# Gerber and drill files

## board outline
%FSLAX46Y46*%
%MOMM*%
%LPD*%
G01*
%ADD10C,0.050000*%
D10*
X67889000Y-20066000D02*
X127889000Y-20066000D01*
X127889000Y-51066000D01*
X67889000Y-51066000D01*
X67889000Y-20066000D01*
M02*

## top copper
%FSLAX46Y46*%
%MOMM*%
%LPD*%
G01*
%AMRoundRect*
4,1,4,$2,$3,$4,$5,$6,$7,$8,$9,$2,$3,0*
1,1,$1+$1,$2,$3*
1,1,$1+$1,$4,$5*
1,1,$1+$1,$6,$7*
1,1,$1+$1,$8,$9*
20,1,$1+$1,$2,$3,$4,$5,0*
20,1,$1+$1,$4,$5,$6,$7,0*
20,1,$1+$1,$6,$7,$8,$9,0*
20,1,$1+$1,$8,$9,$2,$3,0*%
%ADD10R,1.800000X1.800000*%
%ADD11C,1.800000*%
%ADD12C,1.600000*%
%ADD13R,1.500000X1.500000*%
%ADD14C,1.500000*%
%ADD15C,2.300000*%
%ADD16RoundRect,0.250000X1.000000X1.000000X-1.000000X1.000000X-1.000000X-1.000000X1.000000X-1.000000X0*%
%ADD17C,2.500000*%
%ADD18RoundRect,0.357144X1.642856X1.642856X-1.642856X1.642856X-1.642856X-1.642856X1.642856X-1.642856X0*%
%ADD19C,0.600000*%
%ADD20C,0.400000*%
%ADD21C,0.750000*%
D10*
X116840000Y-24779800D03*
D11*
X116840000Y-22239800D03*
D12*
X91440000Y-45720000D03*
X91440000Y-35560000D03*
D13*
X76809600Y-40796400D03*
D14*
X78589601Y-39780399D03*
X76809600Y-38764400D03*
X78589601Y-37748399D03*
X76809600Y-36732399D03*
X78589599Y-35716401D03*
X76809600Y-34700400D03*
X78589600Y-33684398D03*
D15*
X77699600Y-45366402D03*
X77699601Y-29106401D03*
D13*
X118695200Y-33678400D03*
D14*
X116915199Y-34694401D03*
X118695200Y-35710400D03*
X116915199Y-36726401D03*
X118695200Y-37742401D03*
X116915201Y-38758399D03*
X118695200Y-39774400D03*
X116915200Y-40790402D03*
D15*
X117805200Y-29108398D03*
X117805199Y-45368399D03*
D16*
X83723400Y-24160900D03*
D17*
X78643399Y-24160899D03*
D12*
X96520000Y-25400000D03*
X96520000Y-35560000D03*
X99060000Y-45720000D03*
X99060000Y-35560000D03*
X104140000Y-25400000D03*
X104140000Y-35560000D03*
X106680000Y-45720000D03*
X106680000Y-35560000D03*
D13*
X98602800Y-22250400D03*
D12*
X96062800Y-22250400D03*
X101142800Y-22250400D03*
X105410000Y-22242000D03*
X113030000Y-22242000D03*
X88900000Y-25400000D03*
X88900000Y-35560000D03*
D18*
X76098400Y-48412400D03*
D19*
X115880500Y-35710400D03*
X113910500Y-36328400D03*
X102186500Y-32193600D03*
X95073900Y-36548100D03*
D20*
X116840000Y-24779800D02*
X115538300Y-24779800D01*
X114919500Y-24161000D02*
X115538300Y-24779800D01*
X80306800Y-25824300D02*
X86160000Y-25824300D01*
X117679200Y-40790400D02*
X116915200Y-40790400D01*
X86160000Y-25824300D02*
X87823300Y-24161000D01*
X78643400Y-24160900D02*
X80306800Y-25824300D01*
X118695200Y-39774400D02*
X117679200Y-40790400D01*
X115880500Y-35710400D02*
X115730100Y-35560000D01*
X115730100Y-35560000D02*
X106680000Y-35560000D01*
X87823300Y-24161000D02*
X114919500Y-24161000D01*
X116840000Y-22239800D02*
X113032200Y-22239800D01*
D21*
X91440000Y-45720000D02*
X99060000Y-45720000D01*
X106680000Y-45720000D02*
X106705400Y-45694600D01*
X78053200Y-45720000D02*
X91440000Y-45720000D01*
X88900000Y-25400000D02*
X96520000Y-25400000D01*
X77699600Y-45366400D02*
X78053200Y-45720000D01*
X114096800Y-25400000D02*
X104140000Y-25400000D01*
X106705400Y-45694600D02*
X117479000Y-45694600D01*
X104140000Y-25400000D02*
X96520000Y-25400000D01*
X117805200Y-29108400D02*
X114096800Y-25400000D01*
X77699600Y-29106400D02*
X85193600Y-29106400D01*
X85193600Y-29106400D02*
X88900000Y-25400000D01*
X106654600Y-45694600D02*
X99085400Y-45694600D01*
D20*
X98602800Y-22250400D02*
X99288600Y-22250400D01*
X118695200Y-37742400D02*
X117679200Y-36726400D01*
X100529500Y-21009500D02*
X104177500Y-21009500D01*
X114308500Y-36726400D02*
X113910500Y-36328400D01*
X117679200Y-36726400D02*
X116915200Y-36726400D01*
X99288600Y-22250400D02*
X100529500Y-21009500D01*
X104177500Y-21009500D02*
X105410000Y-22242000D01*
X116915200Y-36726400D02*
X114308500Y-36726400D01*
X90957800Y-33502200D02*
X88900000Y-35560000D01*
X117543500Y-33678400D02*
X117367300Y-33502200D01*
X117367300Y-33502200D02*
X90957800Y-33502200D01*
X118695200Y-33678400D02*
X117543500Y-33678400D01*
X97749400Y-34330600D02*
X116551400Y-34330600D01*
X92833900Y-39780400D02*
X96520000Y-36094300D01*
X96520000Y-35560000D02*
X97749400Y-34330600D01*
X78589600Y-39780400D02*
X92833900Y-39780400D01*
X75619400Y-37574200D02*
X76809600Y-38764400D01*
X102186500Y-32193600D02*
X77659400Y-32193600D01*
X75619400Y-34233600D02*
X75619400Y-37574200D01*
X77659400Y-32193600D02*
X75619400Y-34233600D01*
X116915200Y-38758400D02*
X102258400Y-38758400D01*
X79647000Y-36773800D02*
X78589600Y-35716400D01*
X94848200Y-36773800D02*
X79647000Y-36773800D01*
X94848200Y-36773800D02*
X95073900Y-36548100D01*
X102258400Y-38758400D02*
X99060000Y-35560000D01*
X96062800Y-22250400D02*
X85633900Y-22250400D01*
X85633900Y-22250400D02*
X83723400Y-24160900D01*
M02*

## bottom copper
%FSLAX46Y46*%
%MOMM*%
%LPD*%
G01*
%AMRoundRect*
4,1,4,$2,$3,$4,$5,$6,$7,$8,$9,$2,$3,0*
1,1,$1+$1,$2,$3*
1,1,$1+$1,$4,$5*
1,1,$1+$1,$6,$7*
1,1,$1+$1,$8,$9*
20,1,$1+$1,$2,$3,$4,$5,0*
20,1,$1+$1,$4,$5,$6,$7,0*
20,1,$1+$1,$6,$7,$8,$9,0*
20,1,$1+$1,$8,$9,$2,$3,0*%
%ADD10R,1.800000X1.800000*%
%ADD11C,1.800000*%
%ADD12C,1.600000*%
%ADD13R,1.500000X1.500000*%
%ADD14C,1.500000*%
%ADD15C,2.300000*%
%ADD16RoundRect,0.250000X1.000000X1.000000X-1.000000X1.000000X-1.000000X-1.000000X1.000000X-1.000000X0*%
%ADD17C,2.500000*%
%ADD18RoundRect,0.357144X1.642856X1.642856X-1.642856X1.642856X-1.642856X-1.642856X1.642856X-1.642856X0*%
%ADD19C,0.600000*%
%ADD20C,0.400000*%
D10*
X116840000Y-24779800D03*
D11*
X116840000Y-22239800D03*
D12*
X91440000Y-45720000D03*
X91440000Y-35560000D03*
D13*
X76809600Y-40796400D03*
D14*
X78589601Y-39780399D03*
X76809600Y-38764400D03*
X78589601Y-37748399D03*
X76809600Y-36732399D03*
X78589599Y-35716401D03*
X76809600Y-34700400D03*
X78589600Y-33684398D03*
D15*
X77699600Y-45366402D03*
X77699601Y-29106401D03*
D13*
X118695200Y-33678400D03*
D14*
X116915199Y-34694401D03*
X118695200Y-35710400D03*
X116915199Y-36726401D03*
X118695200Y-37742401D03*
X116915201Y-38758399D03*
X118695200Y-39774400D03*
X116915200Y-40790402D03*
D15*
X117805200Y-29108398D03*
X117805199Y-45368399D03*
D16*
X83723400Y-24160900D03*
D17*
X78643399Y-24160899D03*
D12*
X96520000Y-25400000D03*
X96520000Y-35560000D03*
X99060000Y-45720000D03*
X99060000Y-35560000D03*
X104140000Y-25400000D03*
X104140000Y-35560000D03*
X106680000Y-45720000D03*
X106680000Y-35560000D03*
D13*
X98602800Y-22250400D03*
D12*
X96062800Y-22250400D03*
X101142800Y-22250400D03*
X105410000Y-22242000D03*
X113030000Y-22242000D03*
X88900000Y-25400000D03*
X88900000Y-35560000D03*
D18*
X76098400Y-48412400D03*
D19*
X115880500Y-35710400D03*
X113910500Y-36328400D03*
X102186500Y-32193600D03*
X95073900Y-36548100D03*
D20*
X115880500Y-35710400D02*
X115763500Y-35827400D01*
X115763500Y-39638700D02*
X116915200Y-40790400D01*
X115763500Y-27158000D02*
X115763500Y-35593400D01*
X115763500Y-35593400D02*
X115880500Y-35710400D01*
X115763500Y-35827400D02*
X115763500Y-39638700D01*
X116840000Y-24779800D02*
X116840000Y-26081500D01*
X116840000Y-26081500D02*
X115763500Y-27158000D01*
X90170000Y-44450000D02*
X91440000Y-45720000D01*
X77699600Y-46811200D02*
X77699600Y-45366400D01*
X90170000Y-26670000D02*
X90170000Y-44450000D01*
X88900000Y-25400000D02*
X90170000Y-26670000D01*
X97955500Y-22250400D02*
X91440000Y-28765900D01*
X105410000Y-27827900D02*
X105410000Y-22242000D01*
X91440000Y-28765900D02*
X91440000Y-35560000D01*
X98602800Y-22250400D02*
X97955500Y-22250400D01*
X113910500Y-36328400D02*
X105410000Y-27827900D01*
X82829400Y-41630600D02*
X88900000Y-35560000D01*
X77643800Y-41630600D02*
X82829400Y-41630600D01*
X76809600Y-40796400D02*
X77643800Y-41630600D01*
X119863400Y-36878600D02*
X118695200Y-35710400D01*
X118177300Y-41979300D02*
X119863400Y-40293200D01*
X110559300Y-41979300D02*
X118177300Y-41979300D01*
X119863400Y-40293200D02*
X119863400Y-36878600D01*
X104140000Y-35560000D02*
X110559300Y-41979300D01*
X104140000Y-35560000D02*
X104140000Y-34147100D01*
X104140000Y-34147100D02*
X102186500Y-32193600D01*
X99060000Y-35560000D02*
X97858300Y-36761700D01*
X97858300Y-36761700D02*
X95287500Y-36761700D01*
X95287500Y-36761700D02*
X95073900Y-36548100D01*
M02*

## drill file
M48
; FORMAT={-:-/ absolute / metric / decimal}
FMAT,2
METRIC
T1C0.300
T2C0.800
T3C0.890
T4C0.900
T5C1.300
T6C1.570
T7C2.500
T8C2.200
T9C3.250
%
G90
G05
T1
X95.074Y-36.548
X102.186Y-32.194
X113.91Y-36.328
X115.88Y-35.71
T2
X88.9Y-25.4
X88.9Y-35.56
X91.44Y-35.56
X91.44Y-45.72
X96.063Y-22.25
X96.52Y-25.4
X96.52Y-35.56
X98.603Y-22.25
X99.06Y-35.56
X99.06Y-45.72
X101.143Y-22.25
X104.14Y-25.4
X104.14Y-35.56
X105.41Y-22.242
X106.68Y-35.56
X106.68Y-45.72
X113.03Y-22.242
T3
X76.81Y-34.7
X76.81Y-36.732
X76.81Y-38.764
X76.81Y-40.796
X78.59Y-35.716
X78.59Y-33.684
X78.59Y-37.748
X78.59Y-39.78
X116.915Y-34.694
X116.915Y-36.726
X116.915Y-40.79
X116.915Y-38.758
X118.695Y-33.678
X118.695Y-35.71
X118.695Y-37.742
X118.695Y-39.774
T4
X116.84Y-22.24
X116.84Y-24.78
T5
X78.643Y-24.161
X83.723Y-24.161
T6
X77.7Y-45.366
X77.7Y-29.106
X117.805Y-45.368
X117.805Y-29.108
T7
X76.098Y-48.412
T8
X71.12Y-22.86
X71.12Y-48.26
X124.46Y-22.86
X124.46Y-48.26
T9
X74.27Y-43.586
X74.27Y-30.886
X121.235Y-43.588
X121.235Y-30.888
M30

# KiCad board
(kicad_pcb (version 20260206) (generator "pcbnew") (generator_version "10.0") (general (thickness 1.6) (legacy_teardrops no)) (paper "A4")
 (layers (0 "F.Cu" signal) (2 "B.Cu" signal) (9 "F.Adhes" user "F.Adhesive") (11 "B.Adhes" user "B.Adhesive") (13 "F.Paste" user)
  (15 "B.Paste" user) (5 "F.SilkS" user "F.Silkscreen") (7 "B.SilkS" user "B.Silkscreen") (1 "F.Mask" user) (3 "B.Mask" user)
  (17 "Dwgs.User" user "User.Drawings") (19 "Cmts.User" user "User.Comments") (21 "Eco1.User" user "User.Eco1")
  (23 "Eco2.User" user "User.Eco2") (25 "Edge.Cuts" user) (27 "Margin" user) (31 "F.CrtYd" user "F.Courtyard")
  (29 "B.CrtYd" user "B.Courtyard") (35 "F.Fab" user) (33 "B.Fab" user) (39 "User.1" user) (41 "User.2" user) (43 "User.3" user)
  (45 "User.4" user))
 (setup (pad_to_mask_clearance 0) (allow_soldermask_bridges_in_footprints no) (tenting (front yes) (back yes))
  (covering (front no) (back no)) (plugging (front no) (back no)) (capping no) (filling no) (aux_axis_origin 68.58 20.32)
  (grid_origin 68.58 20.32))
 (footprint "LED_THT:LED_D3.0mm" (layer "F.Cu") (at 116.84 24.7798 90)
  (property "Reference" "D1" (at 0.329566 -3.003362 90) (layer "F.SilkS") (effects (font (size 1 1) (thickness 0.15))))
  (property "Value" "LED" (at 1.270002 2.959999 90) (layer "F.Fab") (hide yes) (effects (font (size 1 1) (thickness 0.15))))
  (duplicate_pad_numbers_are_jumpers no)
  (pad "1" thru_hole rect (at 0 0 90) (size 1.8 1.8) (drill 0.9) (layers "*.Cu" "*.Mask") (remove_unused_layers no) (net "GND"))
  (pad "2" thru_hole circle (at 2.54 0 90) (size 1.8 1.8) (drill 0.9) (layers "*.Cu" "*.Mask") (remove_unused_layers no) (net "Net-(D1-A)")))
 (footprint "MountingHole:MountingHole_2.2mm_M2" (layer "F.Cu") (at 124.46 22.86)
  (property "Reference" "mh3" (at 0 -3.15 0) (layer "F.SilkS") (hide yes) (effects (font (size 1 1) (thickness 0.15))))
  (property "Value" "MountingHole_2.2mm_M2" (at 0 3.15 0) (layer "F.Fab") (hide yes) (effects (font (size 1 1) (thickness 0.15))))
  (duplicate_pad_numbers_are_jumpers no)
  (pad "" np_thru_hole circle (at 0 0) (size 2.2 2.2) (drill 2.2) (layers "*.Cu" "*.Mask")))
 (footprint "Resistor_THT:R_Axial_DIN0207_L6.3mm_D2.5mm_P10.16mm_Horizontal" (layer "F.Cu") (at 91.44 45.72 90)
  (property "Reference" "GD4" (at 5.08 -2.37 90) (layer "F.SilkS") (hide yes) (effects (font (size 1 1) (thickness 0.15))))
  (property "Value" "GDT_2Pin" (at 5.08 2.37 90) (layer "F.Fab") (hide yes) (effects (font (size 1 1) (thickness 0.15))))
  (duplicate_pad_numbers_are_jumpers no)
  (pad "1" thru_hole circle (at 0 0 90) (size 1.6 1.6) (drill 0.8) (layers "*.Cu" "*.Mask") (remove_unused_layers no) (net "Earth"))
  (pad "2" thru_hole circle (at 10.16 0 90) (size 1.6 1.6) (drill 0.8) (layers "*.Cu" "*.Mask") (remove_unused_layers no)
   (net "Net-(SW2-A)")))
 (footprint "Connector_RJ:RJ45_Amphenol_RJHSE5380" (layer "F.Cu") (at 76.8096 40.7964 90)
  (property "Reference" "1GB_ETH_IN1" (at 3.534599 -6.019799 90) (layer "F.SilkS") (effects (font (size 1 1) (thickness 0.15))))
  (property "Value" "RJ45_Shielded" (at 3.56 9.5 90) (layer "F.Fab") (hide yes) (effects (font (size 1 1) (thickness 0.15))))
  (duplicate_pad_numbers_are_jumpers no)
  (pad "" np_thru_hole circle (at -2.79 -2.54 90) (size 3.25 3.25) (drill 3.25) (layers "*.Cu" "*.Mask"))
  (pad "" np_thru_hole circle (at 9.909999 -2.539999 90) (size 3.25 3.25) (drill 3.25) (layers "*.Cu" "*.Mask"))
  (pad "1" thru_hole rect (at 0 0 90) (size 1.5 1.5) (drill 0.89) (layers "*.Cu" "*.Mask") (remove_unused_layers no)
   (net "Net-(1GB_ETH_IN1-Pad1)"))
  (pad "2" thru_hole circle (at 1.016001 1.780001 90) (size 1.5 1.5) (drill 0.89) (layers "*.Cu" "*.Mask") (remove_unused_layers no)
   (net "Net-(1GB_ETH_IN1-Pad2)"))
  (pad "3" thru_hole circle (at 2.032 0 90) (size 1.5 1.5) (drill 0.89) (layers "*.Cu" "*.Mask") (remove_unused_layers no)
   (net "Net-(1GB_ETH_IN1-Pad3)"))
  (pad "4" thru_hole circle (at 3.048001 1.780001 90) (size 1.5 1.5) (drill 0.89) (layers "*.Cu" "*.Mask") (remove_unused_layers no)
   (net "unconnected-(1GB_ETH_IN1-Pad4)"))
  (pad "5" thru_hole circle (at 4.064001 0 90) (size 1.5 1.5) (drill 0.89) (layers "*.Cu" "*.Mask") (remove_unused_layers no)
   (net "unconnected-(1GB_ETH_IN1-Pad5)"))
  (pad "6" thru_hole circle (at 5.079999 1.779999 90) (size 1.5 1.5) (drill 0.89) (layers "*.Cu" "*.Mask") (remove_unused_layers no)
   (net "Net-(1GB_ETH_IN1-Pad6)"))
  (pad "7" thru_hole circle (at 6.096 0 90) (size 1.5 1.5) (drill 0.89) (layers "*.Cu" "*.Mask") (remove_unused_layers no)
   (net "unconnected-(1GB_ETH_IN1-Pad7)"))
  (pad "8" thru_hole circle (at 7.112002 1.78 90) (size 1.5 1.5) (drill 0.89) (layers "*.Cu" "*.Mask") (remove_unused_layers no)
   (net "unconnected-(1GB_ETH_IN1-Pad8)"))
  (pad "SH" thru_hole circle (at -4.570002 0.89 90) (size 2.3 2.3) (drill 1.57) (layers "*.Cu" "*.Mask") (remove_unused_layers no)
   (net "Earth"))
  (pad "SH" thru_hole circle (at 11.689999 0.890001 90) (size 2.3 2.3) (drill 1.57) (layers "*.Cu" "*.Mask") (remove_unused_layers no)
   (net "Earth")))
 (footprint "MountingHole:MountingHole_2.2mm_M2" (layer "F.Cu") (at 124.46 48.26)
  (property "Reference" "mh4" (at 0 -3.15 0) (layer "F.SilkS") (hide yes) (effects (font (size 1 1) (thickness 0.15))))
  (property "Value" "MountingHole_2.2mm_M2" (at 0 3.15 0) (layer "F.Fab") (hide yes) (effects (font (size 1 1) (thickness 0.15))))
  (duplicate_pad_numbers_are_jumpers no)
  (pad "" np_thru_hole circle (at 0 0) (size 2.2 2.2) (drill 2.2) (layers "*.Cu" "*.Mask")))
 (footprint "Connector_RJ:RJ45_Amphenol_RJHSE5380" (layer "F.Cu") (at 118.6952 33.6784 -90)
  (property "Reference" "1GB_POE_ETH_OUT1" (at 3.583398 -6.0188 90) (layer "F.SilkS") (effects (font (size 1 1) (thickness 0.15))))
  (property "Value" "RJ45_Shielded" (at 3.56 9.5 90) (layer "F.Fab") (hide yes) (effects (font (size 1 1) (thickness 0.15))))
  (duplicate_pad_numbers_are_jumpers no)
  (pad "" np_thru_hole circle (at -2.79 -2.54 270) (size 3.25 3.25) (drill 3.25) (layers "*.Cu" "*.Mask"))
  (pad "" np_thru_hole circle (at 9.909999 -2.539999 270) (size 3.25 3.25) (drill 3.25) (layers "*.Cu" "*.Mask"))
  (pad "1" thru_hole rect (at 0 0 270) (size 1.5 1.5) (drill 0.89) (layers "*.Cu" "*.Mask") (remove_unused_layers no)
   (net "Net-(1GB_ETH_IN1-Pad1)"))
  (pad "2" thru_hole circle (at 1.016001 1.780001 270) (size 1.5 1.5) (drill 0.89) (layers "*.Cu" "*.Mask") (remove_unused_layers no)
   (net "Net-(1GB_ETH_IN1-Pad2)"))
  (pad "3" thru_hole circle (at 2.032 0 270) (size 1.5 1.5) (drill 0.89) (layers "*.Cu" "*.Mask") (remove_unused_layers no)
   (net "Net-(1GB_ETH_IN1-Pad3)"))
  (pad "4" thru_hole circle (at 3.048001 1.780001 270) (size 1.5 1.5) (drill 0.89) (layers "*.Cu" "*.Mask") (remove_unused_layers no)
   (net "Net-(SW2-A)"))
  (pad "5" thru_hole circle (at 4.064001 0 270) (size 1.5 1.5) (drill 0.89) (layers "*.Cu" "*.Mask") (remove_unused_layers no)
   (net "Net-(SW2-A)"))
  (pad "6" thru_hole circle (at 5.079999 1.779999 270) (size 1.5 1.5) (drill 0.89) (layers "*.Cu" "*.Mask") (remove_unused_layers no)
   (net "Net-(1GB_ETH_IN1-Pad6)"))
  (pad "7" thru_hole circle (at 6.096 0 270) (size 1.5 1.5) (drill 0.89) (layers "*.Cu" "*.Mask") (remove_unused_layers no) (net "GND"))
  (pad "8" thru_hole circle (at 7.112002 1.78 270) (size 1.5 1.5) (drill 0.89) (layers "*.Cu" "*.Mask") (remove_unused_layers no)
   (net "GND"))
  (pad "SH" thru_hole circle (at -4.570002 0.89 270) (size 2.3 2.3) (drill 1.57) (layers "*.Cu" "*.Mask") (remove_unused_layers no)
   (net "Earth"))
  (pad "SH" thru_hole circle (at 11.689999 0.890001 270) (size 2.3 2.3) (drill 1.57) (layers "*.Cu" "*.Mask") (remove_unused_layers no)
   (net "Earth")))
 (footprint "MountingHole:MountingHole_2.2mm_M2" (layer "F.Cu") (at 71.12 22.86)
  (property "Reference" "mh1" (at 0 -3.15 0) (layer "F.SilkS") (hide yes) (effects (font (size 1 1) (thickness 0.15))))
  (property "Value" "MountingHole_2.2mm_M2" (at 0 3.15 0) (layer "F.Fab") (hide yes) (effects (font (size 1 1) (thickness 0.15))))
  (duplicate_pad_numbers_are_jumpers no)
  (pad "" np_thru_hole circle (at 0 0) (size 2.2 2.2) (drill 2.2) (layers "*.Cu" "*.Mask")))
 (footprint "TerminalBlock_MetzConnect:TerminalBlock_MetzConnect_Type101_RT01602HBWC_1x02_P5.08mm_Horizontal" (layer "F.Cu")
  (at 83.7234 24.1609 180)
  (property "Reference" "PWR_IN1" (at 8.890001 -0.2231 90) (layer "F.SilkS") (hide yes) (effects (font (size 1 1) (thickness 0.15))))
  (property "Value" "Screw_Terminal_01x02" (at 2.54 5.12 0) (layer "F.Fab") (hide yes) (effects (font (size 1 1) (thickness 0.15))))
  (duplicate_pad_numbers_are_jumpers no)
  (pad "1" thru_hole roundrect (at 0 0 180) (size 2.5 2.5) (drill 1.3) (layers "*.Cu" "*.Mask") (remove_unused_layers no)
   (roundrect_rratio 0.1) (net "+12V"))
  (pad "2" thru_hole circle (at 5.080001 0.000001 180) (size 2.5 2.5) (drill 1.3) (layers "*.Cu" "*.Mask") (remove_unused_layers no)
   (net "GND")))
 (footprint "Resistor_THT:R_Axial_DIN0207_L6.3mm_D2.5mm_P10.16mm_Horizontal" (layer "F.Cu") (at 96.52 25.4 -90)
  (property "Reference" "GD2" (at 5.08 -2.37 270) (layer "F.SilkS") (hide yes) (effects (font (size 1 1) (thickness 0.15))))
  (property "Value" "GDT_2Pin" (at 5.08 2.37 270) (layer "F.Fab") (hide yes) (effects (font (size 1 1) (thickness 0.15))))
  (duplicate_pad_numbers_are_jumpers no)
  (pad "1" thru_hole circle (at 0 0 270) (size 1.6 1.6) (drill 0.8) (layers "*.Cu" "*.Mask") (remove_unused_layers no) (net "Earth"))
  (pad "2" thru_hole circle (at 10.16 0 270) (size 1.6 1.6) (drill 0.8) (layers "*.Cu" "*.Mask") (remove_unused_layers no)
   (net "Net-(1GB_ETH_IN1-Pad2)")))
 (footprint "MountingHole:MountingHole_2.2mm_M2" (layer "F.Cu") (at 71.12 48.26)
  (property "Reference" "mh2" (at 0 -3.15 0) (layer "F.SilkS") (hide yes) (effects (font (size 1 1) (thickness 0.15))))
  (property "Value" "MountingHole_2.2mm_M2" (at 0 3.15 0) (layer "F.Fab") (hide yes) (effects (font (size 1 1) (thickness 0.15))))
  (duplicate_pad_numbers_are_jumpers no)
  (pad "" np_thru_hole circle (at 0 0) (size 2.2 2.2) (drill 2.2) (layers "*.Cu" "*.Mask")))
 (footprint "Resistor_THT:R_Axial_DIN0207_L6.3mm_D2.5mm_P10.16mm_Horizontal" (layer "F.Cu") (at 99.06 45.72 90)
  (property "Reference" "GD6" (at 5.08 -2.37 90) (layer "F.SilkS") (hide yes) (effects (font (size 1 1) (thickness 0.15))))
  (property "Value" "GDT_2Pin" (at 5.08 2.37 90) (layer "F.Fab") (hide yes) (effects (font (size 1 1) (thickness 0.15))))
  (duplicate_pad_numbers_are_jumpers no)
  (pad "1" thru_hole circle (at 0 0 90) (size 1.6 1.6) (drill 0.8) (layers "*.Cu" "*.Mask") (remove_unused_layers no) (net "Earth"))
  (pad "2" thru_hole circle (at 10.16 0 90) (size 1.6 1.6) (drill 0.8) (layers "*.Cu" "*.Mask") (remove_unused_layers no)
   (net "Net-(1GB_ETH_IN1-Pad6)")))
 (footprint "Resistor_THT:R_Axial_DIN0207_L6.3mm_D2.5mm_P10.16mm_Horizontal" (layer "F.Cu") (at 104.14 25.4 -90)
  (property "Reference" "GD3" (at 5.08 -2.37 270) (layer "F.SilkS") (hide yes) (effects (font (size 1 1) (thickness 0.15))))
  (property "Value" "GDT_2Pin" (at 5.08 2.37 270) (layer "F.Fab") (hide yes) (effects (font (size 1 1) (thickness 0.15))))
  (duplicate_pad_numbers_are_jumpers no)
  (pad "1" thru_hole circle (at 0 0 270) (size 1.6 1.6) (drill 0.8) (layers "*.Cu" "*.Mask") (remove_unused_layers no) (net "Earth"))
  (pad "2" thru_hole circle (at 10.16 0 270) (size 1.6 1.6) (drill 0.8) (layers "*.Cu" "*.Mask") (remove_unused_layers no)
   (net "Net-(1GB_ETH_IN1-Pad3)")))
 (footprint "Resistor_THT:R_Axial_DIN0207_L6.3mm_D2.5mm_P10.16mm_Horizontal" (layer "F.Cu") (at 106.68 45.72 90)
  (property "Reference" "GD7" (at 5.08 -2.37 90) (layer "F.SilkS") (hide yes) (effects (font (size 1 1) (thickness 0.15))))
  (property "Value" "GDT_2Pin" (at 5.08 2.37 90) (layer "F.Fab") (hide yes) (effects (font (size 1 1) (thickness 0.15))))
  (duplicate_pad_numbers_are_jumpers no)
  (pad "1" thru_hole circle (at 0 0 90) (size 1.6 1.6) (drill 0.8) (layers "*.Cu" "*.Mask") (remove_unused_layers no) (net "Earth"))
  (pad "2" thru_hole circle (at 10.16 0 90) (size 1.6 1.6) (drill 0.8) (layers "*.Cu" "*.Mask") (remove_unused_layers no) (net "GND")))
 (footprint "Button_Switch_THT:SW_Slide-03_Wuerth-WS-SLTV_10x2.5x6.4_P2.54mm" (layer "F.Cu") (at 98.6028 22.2504)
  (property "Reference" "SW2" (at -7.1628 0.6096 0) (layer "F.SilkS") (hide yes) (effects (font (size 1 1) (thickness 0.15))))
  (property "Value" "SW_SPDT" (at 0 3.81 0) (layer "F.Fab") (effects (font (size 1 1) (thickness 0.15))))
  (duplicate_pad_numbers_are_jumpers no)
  (pad "1" thru_hole rect (at 0 0) (size 1.5 1.5) (drill 0.8) (layers "*.Cu" "*.Mask") (remove_unused_layers no) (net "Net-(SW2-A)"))
  (pad "2" thru_hole circle (at -2.54 0) (size 1.6 1.6) (drill 0.8) (layers "*.Cu" "*.Mask") (remove_unused_layers no) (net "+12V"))
  (pad "3" thru_hole circle (at 2.54 0) (size 1.6 1.6) (drill 0.8) (layers "*.Cu" "*.Mask") (remove_unused_layers no)
   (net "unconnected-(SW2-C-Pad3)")))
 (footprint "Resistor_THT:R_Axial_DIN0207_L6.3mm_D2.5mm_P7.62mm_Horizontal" (layer "F.Cu") (at 105.41 22.242)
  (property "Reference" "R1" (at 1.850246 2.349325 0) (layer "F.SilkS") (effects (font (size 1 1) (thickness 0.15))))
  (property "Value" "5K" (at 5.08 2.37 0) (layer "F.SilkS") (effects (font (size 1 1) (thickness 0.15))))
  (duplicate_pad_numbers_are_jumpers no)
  (pad "1" thru_hole circle (at 0 0) (size 1.6 1.6) (drill 0.8) (layers "*.Cu" "*.Mask") (remove_unused_layers no) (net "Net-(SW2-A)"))
  (pad "2" thru_hole circle (at 7.62 0) (size 1.6 1.6) (drill 0.8) (layers "*.Cu" "*.Mask") (remove_unused_layers no) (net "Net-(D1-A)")))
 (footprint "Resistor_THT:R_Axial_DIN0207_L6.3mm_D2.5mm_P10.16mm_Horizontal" (layer "F.Cu") (at 88.9 25.4 -90)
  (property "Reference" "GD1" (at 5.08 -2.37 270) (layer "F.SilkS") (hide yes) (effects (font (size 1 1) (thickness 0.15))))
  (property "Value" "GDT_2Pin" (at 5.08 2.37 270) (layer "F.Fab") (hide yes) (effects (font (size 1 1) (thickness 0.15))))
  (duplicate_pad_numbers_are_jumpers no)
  (pad "1" thru_hole circle (at 0 0 270) (size 1.6 1.6) (drill 0.8) (layers "*.Cu" "*.Mask") (remove_unused_layers no) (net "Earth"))
  (pad "2" thru_hole circle (at 10.16 0 270) (size 1.6 1.6) (drill 0.8) (layers "*.Cu" "*.Mask") (remove_unused_layers no)
   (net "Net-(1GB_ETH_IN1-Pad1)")))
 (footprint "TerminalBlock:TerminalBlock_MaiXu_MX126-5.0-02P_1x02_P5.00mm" (layer "B.Cu") (at 76.0984 48.4124 180)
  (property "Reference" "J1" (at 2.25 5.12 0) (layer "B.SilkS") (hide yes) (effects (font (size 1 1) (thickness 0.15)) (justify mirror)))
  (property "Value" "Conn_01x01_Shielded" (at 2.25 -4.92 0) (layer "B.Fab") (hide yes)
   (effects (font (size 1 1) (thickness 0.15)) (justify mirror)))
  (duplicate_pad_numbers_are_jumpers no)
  (pad "1" thru_hole roundrect (at 0 0 180) (size 4 4) (drill 2.5) (layers "*.Cu" "*.Mask") (remove_unused_layers yes) (keep_end_layers yes)
   (zone_layer_connections) (roundrect_rratio 0.089286) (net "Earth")))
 (gr_rect (start 67.889 20.066) (end 127.889 51.066) (stroke (width 0.05) (type solid)) (fill no) (layer "Edge.Cuts"))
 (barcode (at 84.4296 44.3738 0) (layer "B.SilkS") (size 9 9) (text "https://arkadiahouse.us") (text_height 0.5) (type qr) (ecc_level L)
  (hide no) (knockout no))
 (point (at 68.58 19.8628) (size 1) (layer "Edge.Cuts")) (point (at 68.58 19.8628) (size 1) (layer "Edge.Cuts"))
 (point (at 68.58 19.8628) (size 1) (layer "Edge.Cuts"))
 (segment (start 116.84 24.7798) (end 115.5383 24.7798) (width 0.4) (layer "F.Cu") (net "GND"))
 (segment (start 114.9195 24.161) (end 115.5383 24.7798) (width 0.4) (layer "F.Cu") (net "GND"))
 (segment (start 80.3068 25.8243) (end 86.16 25.8243) (width 0.4) (layer "F.Cu") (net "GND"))
 (segment (start 117.6792 40.7904) (end 116.9152 40.7904) (width 0.4) (layer "F.Cu") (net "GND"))
 (segment (start 86.16 25.8243) (end 87.8233 24.161) (width 0.4) (layer "F.Cu") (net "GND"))
 (segment (start 78.6434 24.1609) (end 80.3068 25.8243) (width 0.4) (layer "F.Cu") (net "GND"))
 (segment (start 118.6952 39.7744) (end 117.6792 40.7904) (width 0.4) (layer "F.Cu") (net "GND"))
 (segment (start 115.8805 35.7104) (end 115.7301 35.56) (width 0.4) (layer "F.Cu") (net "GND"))
 (segment (start 115.7301 35.56) (end 106.68 35.56) (width 0.4) (layer "F.Cu") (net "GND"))
 (segment (start 87.8233 24.161) (end 114.9195 24.161) (width 0.4) (layer "F.Cu") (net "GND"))
 (via (at 115.8805 35.7104) (size 0.6) (drill 0.3) (layers "F.Cu" "B.Cu") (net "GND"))
 (segment (start 115.8805 35.7104) (end 115.7635 35.8274) (width 0.4) (layer "B.Cu") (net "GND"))
 (segment (start 115.7635 39.6387) (end 116.9152 40.7904) (width 0.4) (layer "B.Cu") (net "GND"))
 (segment (start 115.7635 27.158) (end 115.7635 35.5934) (width 0.4) (layer "B.Cu") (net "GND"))
 (segment (start 115.7635 35.5934) (end 115.8805 35.7104) (width 0.4) (layer "B.Cu") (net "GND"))
 (segment (start 115.7635 35.8274) (end 115.7635 39.6387) (width 0.4) (layer "B.Cu") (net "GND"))
 (segment (start 116.84 24.7798) (end 116.84 26.0815) (width 0.4) (layer "B.Cu") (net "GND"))
 (segment (start 116.84 26.0815) (end 115.7635 27.158) (width 0.4) (layer "B.Cu") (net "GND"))
 (segment (start 116.84 22.2398) (end 113.0322 22.2398) (width 0.4) (layer "F.Cu") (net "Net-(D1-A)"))
 (segment (start 91.44 45.72) (end 99.06 45.72) (width 0.75) (layer "F.Cu") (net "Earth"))
 (segment (start 106.68 45.72) (end 106.7054 45.6946) (width 0.75) (layer "F.Cu") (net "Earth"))
 (segment (start 78.0532 45.72) (end 91.44 45.72) (width 0.75) (layer "F.Cu") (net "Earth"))
 (segment (start 88.9 25.4) (end 96.52 25.4) (width 0.75) (layer "F.Cu") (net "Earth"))
 (segment (start 77.6996 45.3664) (end 78.0532 45.72) (width 0.75) (layer "F.Cu") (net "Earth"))
 (segment (start 114.0968 25.4) (end 104.14 25.4) (width 0.75) (layer "F.Cu") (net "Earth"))
 (segment (start 106.7054 45.6946) (end 117.479 45.6946) (width 0.75) (layer "F.Cu") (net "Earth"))
 (segment (start 104.14 25.4) (end 96.52 25.4) (width 0.75) (layer "F.Cu") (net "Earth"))
 (segment (start 117.8052 29.1084) (end 114.0968 25.4) (width 0.75) (layer "F.Cu") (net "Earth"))
 (segment (start 77.6996 29.1064) (end 85.1936 29.1064) (width 0.75) (layer "F.Cu") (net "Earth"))
 (segment (start 85.1936 29.1064) (end 88.9 25.4) (width 0.75) (layer "F.Cu") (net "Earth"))
 (segment (start 106.6546 45.6946) (end 99.0854 45.6946) (width 0.75) (layer "F.Cu") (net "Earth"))
 (segment (start 90.17 44.45) (end 91.44 45.72) (width 0.4) (layer "B.Cu") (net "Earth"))
 (segment (start 77.6996 46.8112) (end 77.6996 45.3664) (width 0.4) (layer "B.Cu") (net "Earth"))
 (segment (start 90.17 26.67) (end 90.17 44.45) (width 0.4) (layer "B.Cu") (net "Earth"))
 (segment (start 88.9 25.4) (end 90.17 26.67) (width 0.4) (layer "B.Cu") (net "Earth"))
 (segment (start 98.6028 22.2504) (end 99.2886 22.2504) (width 0.4) (layer "F.Cu") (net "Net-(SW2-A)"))
 (segment (start 118.6952 37.7424) (end 117.6792 36.7264) (width 0.4) (layer "F.Cu") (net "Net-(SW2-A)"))
 (segment (start 100.5295 21.0095) (end 104.1775 21.0095) (width 0.4) (layer "F.Cu") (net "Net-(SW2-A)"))
 (segment (start 114.3085 36.7264) (end 113.9105 36.3284) (width 0.4) (layer "F.Cu") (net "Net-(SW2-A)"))
 (segment (start 117.6792 36.7264) (end 116.9152 36.7264) (width 0.4) (layer "F.Cu") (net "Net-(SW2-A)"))
 (segment (start 99.2886 22.2504) (end 100.5295 21.0095) (width 0.4) (layer "F.Cu") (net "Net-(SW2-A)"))
 (segment (start 104.1775 21.0095) (end 105.41 22.242) (width 0.4) (layer "F.Cu") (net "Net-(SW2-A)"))
 (segment (start 116.9152 36.7264) (end 114.3085 36.7264) (width 0.4) (layer "F.Cu") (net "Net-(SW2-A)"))
 (via (at 113.9105 36.3284) (size 0.6) (drill 0.3) (layers "F.Cu" "B.Cu") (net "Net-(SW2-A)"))
 (segment (start 97.9555 22.2504) (end 91.44 28.7659) (width 0.4) (layer "B.Cu") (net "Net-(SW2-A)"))
 (segment (start 105.41 27.8279) (end 105.41 22.242) (width 0.4) (layer "B.Cu") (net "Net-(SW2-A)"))
 (segment (start 91.44 28.7659) (end 91.44 35.56) (width 0.4) (layer "B.Cu") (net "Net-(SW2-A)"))
 (segment (start 98.6028 22.2504) (end 97.9555 22.2504) (width 0.4) (layer "B.Cu") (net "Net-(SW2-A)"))
 (segment (start 113.9105 36.3284) (end 105.41 27.8279) (width 0.4) (layer "B.Cu") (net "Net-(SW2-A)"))
 (segment (start 90.9578 33.5022) (end 88.9 35.56) (width 0.4) (layer "F.Cu") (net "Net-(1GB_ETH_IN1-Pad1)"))
 (segment (start 117.5435 33.6784) (end 117.3673 33.5022) (width 0.4) (layer "F.Cu") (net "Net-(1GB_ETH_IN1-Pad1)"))
 (segment (start 117.3673 33.5022) (end 90.9578 33.5022) (width 0.4) (layer "F.Cu") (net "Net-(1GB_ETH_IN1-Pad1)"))
 (segment (start 118.6952 33.6784) (end 117.5435 33.6784) (width 0.4) (layer "F.Cu") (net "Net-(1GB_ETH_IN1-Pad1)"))
 (segment (start 82.8294 41.6306) (end 88.9 35.56) (width 0.4) (layer "B.Cu") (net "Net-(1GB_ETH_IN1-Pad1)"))
 (segment (start 77.6438 41.6306) (end 82.8294 41.6306) (width 0.4) (layer "B.Cu") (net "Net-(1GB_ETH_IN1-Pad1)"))
 (segment (start 76.8096 40.7964) (end 77.6438 41.6306) (width 0.4) (layer "B.Cu") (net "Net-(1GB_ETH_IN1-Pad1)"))
 (segment (start 97.7494 34.3306) (end 116.5514 34.3306) (width 0.4) (layer "F.Cu") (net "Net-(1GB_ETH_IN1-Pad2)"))
 (segment (start 92.8339 39.7804) (end 96.52 36.0943) (width 0.4) (layer "F.Cu") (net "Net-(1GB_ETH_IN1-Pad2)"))
 (segment (start 96.52 35.56) (end 97.7494 34.3306) (width 0.4) (layer "F.Cu") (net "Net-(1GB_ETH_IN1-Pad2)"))
 (segment (start 78.5896 39.7804) (end 92.8339 39.7804) (width 0.4) (layer "F.Cu") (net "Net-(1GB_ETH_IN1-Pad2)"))
 (segment (start 75.6194 37.5742) (end 76.8096 38.7644) (width 0.4) (layer "F.Cu") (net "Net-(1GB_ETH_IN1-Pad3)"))
 (segment (start 102.1865 32.1936) (end 77.6594 32.1936) (width 0.4) (layer "F.Cu") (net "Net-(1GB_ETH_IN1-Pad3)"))
 (segment (start 75.6194 34.2336) (end 75.6194 37.5742) (width 0.4) (layer "F.Cu") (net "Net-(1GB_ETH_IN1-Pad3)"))
 (segment (start 77.6594 32.1936) (end 75.6194 34.2336) (width 0.4) (layer "F.Cu") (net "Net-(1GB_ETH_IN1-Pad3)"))
 (via (at 102.1865 32.1936) (size 0.6) (drill 0.3) (layers "F.Cu" "B.Cu") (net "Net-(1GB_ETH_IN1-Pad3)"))
 (segment (start 119.8634 36.8786) (end 118.6952 35.7104) (width 0.4) (layer "B.Cu") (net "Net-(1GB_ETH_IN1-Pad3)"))
 (segment (start 118.1773 41.9793) (end 119.8634 40.2932) (width 0.4) (layer "B.Cu") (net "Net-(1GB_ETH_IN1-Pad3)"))
 (segment (start 110.5593 41.9793) (end 118.1773 41.9793) (width 0.4) (layer "B.Cu") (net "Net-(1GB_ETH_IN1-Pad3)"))
 (segment (start 119.8634 40.2932) (end 119.8634 36.8786) (width 0.4) (layer "B.Cu") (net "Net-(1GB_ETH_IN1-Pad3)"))
 (segment (start 104.14 35.56) (end 110.5593 41.9793) (width 0.4) (layer "B.Cu") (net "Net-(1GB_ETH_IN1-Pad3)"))
 (segment (start 104.14 35.56) (end 104.14 34.1471) (width 0.4) (layer "B.Cu") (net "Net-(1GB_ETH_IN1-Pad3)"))
 (segment (start 104.14 34.1471) (end 102.1865 32.1936) (width 0.4) (layer "B.Cu") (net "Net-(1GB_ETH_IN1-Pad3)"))
 (segment (start 116.9152 38.7584) (end 102.2584 38.7584) (width 0.4) (layer "F.Cu") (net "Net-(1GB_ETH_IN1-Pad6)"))
 (segment (start 79.647 36.7738) (end 78.5896 35.7164) (width 0.4) (layer "F.Cu") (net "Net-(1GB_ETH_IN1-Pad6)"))
 (segment (start 94.8482 36.7738) (end 79.647 36.7738) (width 0.4) (layer "F.Cu") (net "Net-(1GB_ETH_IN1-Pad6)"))
 (segment (start 94.8482 36.7738) (end 95.0739 36.5481) (width 0.4) (layer "F.Cu") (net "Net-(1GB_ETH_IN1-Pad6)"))
 (segment (start 102.2584 38.7584) (end 99.06 35.56) (width 0.4) (layer "F.Cu") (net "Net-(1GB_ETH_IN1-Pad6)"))
 (via (at 95.0739 36.5481) (size 0.6) (drill 0.3) (layers "F.Cu" "B.Cu") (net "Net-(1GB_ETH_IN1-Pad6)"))
 (segment (start 99.06 35.56) (end 97.8583 36.7617) (width 0.4) (layer "B.Cu") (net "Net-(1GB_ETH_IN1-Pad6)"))
 (segment (start 97.8583 36.7617) (end 95.2875 36.7617) (width 0.4) (layer "B.Cu") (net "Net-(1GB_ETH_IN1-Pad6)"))
 (segment (start 95.2875 36.7617) (end 95.0739 36.5481) (width 0.4) (layer "B.Cu") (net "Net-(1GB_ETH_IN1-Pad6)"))
 (segment (start 96.0628 22.2504) (end 85.6339 22.2504) (width 0.4) (layer "F.Cu") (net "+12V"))
 (segment (start 85.6339 22.2504) (end 83.7234 24.1609) (width 0.4) (layer "F.Cu") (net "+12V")))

